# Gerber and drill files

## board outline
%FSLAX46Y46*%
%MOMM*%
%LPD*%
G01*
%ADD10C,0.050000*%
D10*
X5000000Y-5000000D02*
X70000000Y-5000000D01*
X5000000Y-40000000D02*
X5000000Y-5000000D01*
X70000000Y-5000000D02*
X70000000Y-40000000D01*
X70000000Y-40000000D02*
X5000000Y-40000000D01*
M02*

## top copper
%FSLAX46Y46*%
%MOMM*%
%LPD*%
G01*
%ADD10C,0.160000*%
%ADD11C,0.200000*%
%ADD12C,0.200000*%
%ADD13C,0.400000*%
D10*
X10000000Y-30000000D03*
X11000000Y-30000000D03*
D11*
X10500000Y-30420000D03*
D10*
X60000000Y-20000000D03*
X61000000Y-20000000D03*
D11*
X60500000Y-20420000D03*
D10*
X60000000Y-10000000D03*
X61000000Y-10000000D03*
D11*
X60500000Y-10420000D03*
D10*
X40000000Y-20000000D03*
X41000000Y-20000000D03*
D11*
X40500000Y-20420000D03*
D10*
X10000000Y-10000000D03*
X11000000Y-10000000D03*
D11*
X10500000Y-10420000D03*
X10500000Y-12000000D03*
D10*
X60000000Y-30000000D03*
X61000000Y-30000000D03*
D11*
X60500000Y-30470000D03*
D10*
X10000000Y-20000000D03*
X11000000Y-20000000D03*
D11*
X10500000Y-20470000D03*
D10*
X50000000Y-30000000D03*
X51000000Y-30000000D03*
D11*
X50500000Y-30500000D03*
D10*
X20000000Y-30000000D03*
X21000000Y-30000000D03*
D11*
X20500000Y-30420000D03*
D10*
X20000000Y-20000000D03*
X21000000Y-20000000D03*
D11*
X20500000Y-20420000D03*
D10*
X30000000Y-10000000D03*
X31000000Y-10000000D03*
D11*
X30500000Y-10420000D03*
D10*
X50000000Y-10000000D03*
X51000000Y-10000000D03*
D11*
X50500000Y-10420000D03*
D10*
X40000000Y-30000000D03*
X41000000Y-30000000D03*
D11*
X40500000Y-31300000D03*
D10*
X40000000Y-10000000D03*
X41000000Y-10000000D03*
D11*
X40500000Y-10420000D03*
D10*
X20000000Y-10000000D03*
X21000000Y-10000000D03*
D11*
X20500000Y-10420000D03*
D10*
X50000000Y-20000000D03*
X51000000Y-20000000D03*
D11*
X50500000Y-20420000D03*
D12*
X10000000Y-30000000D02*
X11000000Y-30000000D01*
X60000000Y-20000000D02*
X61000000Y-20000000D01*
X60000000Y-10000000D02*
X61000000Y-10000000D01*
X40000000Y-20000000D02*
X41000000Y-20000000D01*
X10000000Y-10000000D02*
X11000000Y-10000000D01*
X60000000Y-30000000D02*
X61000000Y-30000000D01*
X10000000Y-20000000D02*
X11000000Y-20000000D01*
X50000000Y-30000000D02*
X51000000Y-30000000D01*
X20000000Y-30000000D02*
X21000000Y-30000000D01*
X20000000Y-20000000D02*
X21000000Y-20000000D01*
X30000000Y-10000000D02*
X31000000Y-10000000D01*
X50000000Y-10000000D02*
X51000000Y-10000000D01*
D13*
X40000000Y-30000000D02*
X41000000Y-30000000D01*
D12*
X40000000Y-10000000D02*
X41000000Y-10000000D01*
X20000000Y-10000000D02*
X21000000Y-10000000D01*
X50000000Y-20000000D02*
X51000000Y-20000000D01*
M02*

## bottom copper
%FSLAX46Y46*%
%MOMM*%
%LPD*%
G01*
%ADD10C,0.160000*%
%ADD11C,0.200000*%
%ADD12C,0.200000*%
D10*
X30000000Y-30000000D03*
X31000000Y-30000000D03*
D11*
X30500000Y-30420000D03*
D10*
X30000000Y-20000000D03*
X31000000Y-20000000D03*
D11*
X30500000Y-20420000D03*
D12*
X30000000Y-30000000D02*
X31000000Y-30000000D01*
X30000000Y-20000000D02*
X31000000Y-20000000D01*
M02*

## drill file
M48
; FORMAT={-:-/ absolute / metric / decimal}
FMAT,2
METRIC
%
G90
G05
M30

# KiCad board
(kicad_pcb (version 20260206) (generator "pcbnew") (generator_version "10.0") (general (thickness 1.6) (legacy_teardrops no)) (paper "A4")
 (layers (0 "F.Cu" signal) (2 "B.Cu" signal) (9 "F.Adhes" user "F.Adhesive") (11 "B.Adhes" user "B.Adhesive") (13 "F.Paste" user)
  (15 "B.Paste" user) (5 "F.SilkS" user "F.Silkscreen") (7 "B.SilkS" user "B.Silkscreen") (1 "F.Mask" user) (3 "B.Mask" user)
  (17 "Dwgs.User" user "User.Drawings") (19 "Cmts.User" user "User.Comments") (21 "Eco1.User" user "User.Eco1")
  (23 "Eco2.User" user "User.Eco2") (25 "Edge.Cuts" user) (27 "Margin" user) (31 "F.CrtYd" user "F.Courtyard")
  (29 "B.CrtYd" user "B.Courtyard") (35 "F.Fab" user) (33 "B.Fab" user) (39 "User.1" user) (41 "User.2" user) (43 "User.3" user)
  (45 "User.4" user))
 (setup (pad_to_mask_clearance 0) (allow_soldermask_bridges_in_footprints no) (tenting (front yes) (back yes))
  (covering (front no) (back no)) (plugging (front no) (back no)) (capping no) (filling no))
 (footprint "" (layer "F.Cu") (at 10 30)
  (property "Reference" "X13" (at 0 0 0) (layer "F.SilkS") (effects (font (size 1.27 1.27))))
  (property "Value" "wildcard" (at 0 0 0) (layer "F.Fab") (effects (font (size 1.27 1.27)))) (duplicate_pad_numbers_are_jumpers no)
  (pad "1" smd circle (at 0 0) (size 0.16 0.16) (layers "F.Cu") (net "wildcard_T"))
  (pad "2" smd circle (at 1 0) (size 0.16 0.16) (layers "F.Cu") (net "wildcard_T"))
  (pad "3" smd circle (at 0.5 0.42) (size 0.2 0.2) (layers "F.Cu") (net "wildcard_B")))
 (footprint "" (layer "F.Cu") (at 60 20)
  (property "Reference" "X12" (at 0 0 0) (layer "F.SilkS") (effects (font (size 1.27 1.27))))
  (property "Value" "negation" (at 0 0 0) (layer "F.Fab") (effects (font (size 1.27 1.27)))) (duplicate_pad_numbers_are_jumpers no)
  (pad "1" smd circle (at 0 0) (size 0.16 0.16) (layers "F.Cu") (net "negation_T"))
  (pad "2" smd circle (at 1 0) (size 0.16 0.16) (layers "F.Cu") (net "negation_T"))
  (pad "3" smd circle (at 0.5 0.42) (size 0.2 0.2) (layers "F.Cu") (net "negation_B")))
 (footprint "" (layer "F.Cu") (at 60 10)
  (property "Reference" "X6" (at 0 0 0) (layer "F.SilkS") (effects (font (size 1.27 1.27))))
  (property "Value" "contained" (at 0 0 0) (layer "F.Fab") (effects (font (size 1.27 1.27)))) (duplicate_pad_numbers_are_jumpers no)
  (pad "1" smd circle (at 0 0) (size 0.16 0.16) (layers "F.Cu") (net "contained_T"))
  (pad "2" smd circle (at 1 0) (size 0.16 0.16) (layers "F.Cu") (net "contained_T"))
  (pad "3" smd circle (at 0.5 0.42) (size 0.2 0.2) (layers "F.Cu") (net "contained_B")))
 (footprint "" (layer "F.Cu") (at 40 20)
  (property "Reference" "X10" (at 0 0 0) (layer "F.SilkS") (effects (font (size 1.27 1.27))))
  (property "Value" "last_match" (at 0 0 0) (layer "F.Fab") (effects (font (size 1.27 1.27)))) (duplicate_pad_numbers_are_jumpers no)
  (pad "1" smd circle (at 0 0) (size 0.16 0.16) (layers "F.Cu") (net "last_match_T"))
  (pad "2" smd circle (at 1 0) (size 0.16 0.16) (layers "F.Cu") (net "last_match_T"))
  (pad "3" smd circle (at 0.5 0.42) (size 0.2 0.2) (layers "F.Cu") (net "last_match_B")))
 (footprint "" (layer "F.Cu") (at 10 10)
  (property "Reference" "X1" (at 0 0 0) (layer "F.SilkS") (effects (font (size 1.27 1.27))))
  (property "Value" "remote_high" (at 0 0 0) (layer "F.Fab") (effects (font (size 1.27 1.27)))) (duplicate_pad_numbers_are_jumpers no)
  (pad "1" smd circle (at 0 0) (size 0.16 0.16) (layers "F.Cu") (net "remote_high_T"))
  (pad "2" smd circle (at 1 0) (size 0.16 0.16) (layers "F.Cu") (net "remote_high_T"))
  (pad "3" smd circle (at 0.5 0.42) (size 0.2 0.2) (layers "F.Cu") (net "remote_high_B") (clearance 0))
  (pad "4" smd circle (at 0.5 2) (size 0.2 0.2) (layers "F.Cu") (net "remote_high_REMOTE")))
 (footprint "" (layer "F.Cu") (at 60 30)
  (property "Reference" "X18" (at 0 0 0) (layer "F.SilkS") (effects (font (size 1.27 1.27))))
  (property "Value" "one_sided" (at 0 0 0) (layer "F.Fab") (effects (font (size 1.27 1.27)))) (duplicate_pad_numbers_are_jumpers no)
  (pad "1" smd circle (at 0 0) (size 0.16 0.16) (layers "F.Cu") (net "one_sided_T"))
  (pad "2" smd circle (at 1 0) (size 0.16 0.16) (layers "F.Cu") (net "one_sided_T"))
  (pad "3" smd circle (at 0.5 0.47) (size 0.2 0.2) (layers "F.Cu") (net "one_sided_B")))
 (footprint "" (layer "F.Cu") (at 10 20)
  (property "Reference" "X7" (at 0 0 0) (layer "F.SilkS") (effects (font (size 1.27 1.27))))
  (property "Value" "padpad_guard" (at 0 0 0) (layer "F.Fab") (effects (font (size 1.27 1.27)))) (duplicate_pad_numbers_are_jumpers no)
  (pad "1" smd circle (at 0 0) (size 0.16 0.16) (layers "F.Cu") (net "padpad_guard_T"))
  (pad "2" smd circle (at 1 0) (size 0.16 0.16) (layers "F.Cu") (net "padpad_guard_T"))
  (pad "3" smd circle (at 0.5 0.47) (size 0.2 0.2) (layers "F.Cu") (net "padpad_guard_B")))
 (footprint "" (layer "F.Cu") (at 50 30)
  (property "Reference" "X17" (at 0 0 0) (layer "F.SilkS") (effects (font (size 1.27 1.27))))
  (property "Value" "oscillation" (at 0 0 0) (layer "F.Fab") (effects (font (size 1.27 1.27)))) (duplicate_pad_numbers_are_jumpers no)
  (pad "1" smd circle (at 0 0) (size 0.16 0.16) (layers "F.Cu") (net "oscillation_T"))
  (pad "2" smd circle (at 1 0) (size 0.16 0.16) (layers "F.Cu") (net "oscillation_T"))
  (pad "3" smd circle (at 0.5 0.5) (size 0.2 0.2) (layers "F.Cu") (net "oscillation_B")))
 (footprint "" (layer "F.Cu") (at 20 30)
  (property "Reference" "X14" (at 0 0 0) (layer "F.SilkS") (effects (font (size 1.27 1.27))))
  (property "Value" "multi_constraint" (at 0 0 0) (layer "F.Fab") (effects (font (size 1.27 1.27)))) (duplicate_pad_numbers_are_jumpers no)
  (pad "1" smd circle (at 0 0) (size 0.16 0.16) (layers "F.Cu") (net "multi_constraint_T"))
  (pad "2" smd circle (at 1 0) (size 0.16 0.16) (layers "F.Cu") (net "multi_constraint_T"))
  (pad "3" smd circle (at 0.5 0.42) (size 0.2 0.2) (layers "F.Cu") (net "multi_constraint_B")))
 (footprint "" (layer "F.Cu") (at 30 30)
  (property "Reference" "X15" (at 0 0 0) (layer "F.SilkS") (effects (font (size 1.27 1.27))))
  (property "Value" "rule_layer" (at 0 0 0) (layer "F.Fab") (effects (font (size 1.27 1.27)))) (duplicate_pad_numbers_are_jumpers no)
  (pad "1" smd circle (at 0 0) (size 0.16 0.16) (layers "B.Cu") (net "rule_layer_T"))
  (pad "2" smd circle (at 1 0) (size 0.16 0.16) (layers "B.Cu") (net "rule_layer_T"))
  (pad "3" smd circle (at 0.5 0.42) (size 0.2 0.2) (layers "B.Cu") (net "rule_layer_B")))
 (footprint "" (layer "F.Cu") (at 20 20)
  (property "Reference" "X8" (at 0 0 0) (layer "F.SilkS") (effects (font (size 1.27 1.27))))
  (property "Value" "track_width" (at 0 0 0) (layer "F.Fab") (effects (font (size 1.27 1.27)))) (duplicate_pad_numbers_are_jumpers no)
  (pad "1" smd circle (at 0 0) (size 0.16 0.16) (layers "F.Cu") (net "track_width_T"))
  (pad "2" smd circle (at 1 0) (size 0.16 0.16) (layers "F.Cu") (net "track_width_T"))
  (pad "3" smd circle (at 0.5 0.42) (size 0.2 0.2) (layers "F.Cu") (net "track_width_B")))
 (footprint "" (layer "F.Cu") (at 30 10)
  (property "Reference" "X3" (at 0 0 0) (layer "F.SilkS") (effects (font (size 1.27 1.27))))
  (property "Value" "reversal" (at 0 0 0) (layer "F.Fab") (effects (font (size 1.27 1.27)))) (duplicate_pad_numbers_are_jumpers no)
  (pad "1" smd circle (at 0 0) (size 0.16 0.16) (layers "F.Cu") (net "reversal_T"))
  (pad "2" smd circle (at 1 0) (size 0.16 0.16) (layers "F.Cu") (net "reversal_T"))
  (pad "3" smd circle (at 0.5 0.42) (size 0.2 0.2) (layers "F.Cu") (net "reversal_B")))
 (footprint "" (layer "F.Cu") (at 50 10)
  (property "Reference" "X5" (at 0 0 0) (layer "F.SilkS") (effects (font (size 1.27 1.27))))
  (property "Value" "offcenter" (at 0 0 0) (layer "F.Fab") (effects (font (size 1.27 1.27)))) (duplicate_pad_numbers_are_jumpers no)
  (pad "1" smd circle (at 0 0) (size 0.16 0.16) (layers "F.Cu") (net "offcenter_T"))
  (pad "2" smd circle (at 1 0) (size 0.16 0.16) (layers "F.Cu") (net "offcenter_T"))
  (pad "3" smd circle (at 0.5 0.42) (size 0.2 0.2) (layers "F.Cu") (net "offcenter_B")))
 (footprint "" (layer "F.Cu") (at 40 30)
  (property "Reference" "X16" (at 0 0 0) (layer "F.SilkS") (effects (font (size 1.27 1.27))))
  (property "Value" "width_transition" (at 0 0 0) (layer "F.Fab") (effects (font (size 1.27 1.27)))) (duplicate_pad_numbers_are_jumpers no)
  (pad "1" smd circle (at 0 0) (size 0.16 0.16) (layers "F.Cu") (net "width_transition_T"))
  (pad "2" smd circle (at 1 0) (size 0.16 0.16) (layers "F.Cu") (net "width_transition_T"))
  (pad "3" smd circle (at 0.5 1.3) (size 0.2 0.2) (layers "F.Cu") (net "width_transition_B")))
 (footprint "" (layer "F.Cu") (at 30 20)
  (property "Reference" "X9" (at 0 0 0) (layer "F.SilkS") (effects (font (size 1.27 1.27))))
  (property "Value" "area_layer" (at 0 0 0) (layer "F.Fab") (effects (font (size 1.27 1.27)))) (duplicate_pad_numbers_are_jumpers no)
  (pad "1" smd circle (at 0 0) (size 0.16 0.16) (layers "B.Cu") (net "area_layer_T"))
  (pad "2" smd circle (at 1 0) (size 0.16 0.16) (layers "B.Cu") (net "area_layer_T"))
  (pad "3" smd circle (at 0.5 0.42) (size 0.2 0.2) (layers "B.Cu") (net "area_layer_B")))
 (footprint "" (layer "F.Cu") (at 40 10)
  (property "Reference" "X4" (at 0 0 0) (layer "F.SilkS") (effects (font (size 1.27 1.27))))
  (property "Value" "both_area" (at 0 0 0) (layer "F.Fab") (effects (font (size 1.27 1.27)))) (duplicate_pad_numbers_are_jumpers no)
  (pad "1" smd circle (at 0 0) (size 0.16 0.16) (layers "F.Cu") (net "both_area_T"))
  (pad "2" smd circle (at 1 0) (size 0.16 0.16) (layers "F.Cu") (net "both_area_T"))
  (pad "3" smd circle (at 0.5 0.42) (size 0.2 0.2) (layers "F.Cu") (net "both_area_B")))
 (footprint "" (layer "F.Cu") (at 20 10)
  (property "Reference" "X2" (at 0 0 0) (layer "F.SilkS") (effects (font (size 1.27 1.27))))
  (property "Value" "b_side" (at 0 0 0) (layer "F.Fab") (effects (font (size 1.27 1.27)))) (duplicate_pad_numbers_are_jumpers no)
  (pad "1" smd circle (at 0 0) (size 0.16 0.16) (layers "F.Cu") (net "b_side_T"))
  (pad "2" smd circle (at 1 0) (size 0.16 0.16) (layers "F.Cu") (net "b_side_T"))
  (pad "3" smd circle (at 0.5 0.42) (size 0.2 0.2) (layers "F.Cu") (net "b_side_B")))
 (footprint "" (layer "F.Cu") (at 50 20)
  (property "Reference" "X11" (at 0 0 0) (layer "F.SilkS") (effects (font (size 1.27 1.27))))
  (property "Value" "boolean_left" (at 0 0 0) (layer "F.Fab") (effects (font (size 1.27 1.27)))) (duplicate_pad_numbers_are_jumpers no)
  (pad "1" smd circle (at 0 0) (size 0.16 0.16) (layers "F.Cu") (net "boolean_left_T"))
  (pad "2" smd circle (at 1 0) (size 0.16 0.16) (layers "F.Cu") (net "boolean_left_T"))
  (pad "3" smd circle (at 0.5 0.42) (size 0.2 0.2) (layers "F.Cu") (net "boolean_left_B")))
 (gr_line (start 5 5) (end 70 5) (stroke (width 0.05) (type default)) (layer "Edge.Cuts"))
 (gr_line (start 5 40) (end 5 5) (stroke (width 0.05) (type default)) (layer "Edge.Cuts"))
 (gr_line (start 70 5) (end 70 40) (stroke (width 0.05) (type default)) (layer "Edge.Cuts"))
 (gr_line (start 70 40) (end 5 40) (stroke (width 0.05) (type default)) (layer "Edge.Cuts"))
 (segment (start 10 30) (end 11 30) (width 0.2) (layer "F.Cu") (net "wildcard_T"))
 (segment (start 60 20) (end 61 20) (width 0.2) (layer "F.Cu") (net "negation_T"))
 (segment (start 60 10) (end 61 10) (width 0.2) (layer "F.Cu") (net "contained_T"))
 (segment (start 40 20) (end 41 20) (width 0.2) (layer "F.Cu") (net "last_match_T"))
 (segment (start 10 10) (end 11 10) (width 0.2) (layer "F.Cu") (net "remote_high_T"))
 (segment (start 60 30) (end 61 30) (width 0.2) (layer "F.Cu") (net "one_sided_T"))
 (segment (start 10 20) (end 11 20) (width 0.2) (layer "F.Cu") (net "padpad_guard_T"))
 (segment (start 50 30) (end 51 30) (width 0.2) (layer "F.Cu") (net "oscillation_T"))
 (segment (start 20 30) (end 21 30) (width 0.2) (layer "F.Cu") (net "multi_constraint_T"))
 (segment (start 30 30) (end 31 30) (width 0.2) (layer "B.Cu") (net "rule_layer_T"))
 (segment (start 20 20) (end 21 20) (width 0.2) (layer "F.Cu") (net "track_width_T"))
 (segment (start 30 10) (end 31 10) (width 0.2) (layer "F.Cu") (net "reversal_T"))
 (segment (start 50 10) (end 51 10) (width 0.2) (layer "F.Cu") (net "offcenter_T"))
 (segment (start 40 30) (end 41 30) (width 0.4) (layer "F.Cu") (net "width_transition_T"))
 (segment (start 30 20) (end 31 20) (width 0.2) (layer "B.Cu") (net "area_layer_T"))
 (segment (start 40 10) (end 41 10) (width 0.2) (layer "F.Cu") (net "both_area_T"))
 (segment (start 20 10) (end 21 10) (width 0.2) (layer "F.Cu") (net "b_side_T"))
 (segment (start 50 20) (end 51 20) (width 0.2) (layer "F.Cu") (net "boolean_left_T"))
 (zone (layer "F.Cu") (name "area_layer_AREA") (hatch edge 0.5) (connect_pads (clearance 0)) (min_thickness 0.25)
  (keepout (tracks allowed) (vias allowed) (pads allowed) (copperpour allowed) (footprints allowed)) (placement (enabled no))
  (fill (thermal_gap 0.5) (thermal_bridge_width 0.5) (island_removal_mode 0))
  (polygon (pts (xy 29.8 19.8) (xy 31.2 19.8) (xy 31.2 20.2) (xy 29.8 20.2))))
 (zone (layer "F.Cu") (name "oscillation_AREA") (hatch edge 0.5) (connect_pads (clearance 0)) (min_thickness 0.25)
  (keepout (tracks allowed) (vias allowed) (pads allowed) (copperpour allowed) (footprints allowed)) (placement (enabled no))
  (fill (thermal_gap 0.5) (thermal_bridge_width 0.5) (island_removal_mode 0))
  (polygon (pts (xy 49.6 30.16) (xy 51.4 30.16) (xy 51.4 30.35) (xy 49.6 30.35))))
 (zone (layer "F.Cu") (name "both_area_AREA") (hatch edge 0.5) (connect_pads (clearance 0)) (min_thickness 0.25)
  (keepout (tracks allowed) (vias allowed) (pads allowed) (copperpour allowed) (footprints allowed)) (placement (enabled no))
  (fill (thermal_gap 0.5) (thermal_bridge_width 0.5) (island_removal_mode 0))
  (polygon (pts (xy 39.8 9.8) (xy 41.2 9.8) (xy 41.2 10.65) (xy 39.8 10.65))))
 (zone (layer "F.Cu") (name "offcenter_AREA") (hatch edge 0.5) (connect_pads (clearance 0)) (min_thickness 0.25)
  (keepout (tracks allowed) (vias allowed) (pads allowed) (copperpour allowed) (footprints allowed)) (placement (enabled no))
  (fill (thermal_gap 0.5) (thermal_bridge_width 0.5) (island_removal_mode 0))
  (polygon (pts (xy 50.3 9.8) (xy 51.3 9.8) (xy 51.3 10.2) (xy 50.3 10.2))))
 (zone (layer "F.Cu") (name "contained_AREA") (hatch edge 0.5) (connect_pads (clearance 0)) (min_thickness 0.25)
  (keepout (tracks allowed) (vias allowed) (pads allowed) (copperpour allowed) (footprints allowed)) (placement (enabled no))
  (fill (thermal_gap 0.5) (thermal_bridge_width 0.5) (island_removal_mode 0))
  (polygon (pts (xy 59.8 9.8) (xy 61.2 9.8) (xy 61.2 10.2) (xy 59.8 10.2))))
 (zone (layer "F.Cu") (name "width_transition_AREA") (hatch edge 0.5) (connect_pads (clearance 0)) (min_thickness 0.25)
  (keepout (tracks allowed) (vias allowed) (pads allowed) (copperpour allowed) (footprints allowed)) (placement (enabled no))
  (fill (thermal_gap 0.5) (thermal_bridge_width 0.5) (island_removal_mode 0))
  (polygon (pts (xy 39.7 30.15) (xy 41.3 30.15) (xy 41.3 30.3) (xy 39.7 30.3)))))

